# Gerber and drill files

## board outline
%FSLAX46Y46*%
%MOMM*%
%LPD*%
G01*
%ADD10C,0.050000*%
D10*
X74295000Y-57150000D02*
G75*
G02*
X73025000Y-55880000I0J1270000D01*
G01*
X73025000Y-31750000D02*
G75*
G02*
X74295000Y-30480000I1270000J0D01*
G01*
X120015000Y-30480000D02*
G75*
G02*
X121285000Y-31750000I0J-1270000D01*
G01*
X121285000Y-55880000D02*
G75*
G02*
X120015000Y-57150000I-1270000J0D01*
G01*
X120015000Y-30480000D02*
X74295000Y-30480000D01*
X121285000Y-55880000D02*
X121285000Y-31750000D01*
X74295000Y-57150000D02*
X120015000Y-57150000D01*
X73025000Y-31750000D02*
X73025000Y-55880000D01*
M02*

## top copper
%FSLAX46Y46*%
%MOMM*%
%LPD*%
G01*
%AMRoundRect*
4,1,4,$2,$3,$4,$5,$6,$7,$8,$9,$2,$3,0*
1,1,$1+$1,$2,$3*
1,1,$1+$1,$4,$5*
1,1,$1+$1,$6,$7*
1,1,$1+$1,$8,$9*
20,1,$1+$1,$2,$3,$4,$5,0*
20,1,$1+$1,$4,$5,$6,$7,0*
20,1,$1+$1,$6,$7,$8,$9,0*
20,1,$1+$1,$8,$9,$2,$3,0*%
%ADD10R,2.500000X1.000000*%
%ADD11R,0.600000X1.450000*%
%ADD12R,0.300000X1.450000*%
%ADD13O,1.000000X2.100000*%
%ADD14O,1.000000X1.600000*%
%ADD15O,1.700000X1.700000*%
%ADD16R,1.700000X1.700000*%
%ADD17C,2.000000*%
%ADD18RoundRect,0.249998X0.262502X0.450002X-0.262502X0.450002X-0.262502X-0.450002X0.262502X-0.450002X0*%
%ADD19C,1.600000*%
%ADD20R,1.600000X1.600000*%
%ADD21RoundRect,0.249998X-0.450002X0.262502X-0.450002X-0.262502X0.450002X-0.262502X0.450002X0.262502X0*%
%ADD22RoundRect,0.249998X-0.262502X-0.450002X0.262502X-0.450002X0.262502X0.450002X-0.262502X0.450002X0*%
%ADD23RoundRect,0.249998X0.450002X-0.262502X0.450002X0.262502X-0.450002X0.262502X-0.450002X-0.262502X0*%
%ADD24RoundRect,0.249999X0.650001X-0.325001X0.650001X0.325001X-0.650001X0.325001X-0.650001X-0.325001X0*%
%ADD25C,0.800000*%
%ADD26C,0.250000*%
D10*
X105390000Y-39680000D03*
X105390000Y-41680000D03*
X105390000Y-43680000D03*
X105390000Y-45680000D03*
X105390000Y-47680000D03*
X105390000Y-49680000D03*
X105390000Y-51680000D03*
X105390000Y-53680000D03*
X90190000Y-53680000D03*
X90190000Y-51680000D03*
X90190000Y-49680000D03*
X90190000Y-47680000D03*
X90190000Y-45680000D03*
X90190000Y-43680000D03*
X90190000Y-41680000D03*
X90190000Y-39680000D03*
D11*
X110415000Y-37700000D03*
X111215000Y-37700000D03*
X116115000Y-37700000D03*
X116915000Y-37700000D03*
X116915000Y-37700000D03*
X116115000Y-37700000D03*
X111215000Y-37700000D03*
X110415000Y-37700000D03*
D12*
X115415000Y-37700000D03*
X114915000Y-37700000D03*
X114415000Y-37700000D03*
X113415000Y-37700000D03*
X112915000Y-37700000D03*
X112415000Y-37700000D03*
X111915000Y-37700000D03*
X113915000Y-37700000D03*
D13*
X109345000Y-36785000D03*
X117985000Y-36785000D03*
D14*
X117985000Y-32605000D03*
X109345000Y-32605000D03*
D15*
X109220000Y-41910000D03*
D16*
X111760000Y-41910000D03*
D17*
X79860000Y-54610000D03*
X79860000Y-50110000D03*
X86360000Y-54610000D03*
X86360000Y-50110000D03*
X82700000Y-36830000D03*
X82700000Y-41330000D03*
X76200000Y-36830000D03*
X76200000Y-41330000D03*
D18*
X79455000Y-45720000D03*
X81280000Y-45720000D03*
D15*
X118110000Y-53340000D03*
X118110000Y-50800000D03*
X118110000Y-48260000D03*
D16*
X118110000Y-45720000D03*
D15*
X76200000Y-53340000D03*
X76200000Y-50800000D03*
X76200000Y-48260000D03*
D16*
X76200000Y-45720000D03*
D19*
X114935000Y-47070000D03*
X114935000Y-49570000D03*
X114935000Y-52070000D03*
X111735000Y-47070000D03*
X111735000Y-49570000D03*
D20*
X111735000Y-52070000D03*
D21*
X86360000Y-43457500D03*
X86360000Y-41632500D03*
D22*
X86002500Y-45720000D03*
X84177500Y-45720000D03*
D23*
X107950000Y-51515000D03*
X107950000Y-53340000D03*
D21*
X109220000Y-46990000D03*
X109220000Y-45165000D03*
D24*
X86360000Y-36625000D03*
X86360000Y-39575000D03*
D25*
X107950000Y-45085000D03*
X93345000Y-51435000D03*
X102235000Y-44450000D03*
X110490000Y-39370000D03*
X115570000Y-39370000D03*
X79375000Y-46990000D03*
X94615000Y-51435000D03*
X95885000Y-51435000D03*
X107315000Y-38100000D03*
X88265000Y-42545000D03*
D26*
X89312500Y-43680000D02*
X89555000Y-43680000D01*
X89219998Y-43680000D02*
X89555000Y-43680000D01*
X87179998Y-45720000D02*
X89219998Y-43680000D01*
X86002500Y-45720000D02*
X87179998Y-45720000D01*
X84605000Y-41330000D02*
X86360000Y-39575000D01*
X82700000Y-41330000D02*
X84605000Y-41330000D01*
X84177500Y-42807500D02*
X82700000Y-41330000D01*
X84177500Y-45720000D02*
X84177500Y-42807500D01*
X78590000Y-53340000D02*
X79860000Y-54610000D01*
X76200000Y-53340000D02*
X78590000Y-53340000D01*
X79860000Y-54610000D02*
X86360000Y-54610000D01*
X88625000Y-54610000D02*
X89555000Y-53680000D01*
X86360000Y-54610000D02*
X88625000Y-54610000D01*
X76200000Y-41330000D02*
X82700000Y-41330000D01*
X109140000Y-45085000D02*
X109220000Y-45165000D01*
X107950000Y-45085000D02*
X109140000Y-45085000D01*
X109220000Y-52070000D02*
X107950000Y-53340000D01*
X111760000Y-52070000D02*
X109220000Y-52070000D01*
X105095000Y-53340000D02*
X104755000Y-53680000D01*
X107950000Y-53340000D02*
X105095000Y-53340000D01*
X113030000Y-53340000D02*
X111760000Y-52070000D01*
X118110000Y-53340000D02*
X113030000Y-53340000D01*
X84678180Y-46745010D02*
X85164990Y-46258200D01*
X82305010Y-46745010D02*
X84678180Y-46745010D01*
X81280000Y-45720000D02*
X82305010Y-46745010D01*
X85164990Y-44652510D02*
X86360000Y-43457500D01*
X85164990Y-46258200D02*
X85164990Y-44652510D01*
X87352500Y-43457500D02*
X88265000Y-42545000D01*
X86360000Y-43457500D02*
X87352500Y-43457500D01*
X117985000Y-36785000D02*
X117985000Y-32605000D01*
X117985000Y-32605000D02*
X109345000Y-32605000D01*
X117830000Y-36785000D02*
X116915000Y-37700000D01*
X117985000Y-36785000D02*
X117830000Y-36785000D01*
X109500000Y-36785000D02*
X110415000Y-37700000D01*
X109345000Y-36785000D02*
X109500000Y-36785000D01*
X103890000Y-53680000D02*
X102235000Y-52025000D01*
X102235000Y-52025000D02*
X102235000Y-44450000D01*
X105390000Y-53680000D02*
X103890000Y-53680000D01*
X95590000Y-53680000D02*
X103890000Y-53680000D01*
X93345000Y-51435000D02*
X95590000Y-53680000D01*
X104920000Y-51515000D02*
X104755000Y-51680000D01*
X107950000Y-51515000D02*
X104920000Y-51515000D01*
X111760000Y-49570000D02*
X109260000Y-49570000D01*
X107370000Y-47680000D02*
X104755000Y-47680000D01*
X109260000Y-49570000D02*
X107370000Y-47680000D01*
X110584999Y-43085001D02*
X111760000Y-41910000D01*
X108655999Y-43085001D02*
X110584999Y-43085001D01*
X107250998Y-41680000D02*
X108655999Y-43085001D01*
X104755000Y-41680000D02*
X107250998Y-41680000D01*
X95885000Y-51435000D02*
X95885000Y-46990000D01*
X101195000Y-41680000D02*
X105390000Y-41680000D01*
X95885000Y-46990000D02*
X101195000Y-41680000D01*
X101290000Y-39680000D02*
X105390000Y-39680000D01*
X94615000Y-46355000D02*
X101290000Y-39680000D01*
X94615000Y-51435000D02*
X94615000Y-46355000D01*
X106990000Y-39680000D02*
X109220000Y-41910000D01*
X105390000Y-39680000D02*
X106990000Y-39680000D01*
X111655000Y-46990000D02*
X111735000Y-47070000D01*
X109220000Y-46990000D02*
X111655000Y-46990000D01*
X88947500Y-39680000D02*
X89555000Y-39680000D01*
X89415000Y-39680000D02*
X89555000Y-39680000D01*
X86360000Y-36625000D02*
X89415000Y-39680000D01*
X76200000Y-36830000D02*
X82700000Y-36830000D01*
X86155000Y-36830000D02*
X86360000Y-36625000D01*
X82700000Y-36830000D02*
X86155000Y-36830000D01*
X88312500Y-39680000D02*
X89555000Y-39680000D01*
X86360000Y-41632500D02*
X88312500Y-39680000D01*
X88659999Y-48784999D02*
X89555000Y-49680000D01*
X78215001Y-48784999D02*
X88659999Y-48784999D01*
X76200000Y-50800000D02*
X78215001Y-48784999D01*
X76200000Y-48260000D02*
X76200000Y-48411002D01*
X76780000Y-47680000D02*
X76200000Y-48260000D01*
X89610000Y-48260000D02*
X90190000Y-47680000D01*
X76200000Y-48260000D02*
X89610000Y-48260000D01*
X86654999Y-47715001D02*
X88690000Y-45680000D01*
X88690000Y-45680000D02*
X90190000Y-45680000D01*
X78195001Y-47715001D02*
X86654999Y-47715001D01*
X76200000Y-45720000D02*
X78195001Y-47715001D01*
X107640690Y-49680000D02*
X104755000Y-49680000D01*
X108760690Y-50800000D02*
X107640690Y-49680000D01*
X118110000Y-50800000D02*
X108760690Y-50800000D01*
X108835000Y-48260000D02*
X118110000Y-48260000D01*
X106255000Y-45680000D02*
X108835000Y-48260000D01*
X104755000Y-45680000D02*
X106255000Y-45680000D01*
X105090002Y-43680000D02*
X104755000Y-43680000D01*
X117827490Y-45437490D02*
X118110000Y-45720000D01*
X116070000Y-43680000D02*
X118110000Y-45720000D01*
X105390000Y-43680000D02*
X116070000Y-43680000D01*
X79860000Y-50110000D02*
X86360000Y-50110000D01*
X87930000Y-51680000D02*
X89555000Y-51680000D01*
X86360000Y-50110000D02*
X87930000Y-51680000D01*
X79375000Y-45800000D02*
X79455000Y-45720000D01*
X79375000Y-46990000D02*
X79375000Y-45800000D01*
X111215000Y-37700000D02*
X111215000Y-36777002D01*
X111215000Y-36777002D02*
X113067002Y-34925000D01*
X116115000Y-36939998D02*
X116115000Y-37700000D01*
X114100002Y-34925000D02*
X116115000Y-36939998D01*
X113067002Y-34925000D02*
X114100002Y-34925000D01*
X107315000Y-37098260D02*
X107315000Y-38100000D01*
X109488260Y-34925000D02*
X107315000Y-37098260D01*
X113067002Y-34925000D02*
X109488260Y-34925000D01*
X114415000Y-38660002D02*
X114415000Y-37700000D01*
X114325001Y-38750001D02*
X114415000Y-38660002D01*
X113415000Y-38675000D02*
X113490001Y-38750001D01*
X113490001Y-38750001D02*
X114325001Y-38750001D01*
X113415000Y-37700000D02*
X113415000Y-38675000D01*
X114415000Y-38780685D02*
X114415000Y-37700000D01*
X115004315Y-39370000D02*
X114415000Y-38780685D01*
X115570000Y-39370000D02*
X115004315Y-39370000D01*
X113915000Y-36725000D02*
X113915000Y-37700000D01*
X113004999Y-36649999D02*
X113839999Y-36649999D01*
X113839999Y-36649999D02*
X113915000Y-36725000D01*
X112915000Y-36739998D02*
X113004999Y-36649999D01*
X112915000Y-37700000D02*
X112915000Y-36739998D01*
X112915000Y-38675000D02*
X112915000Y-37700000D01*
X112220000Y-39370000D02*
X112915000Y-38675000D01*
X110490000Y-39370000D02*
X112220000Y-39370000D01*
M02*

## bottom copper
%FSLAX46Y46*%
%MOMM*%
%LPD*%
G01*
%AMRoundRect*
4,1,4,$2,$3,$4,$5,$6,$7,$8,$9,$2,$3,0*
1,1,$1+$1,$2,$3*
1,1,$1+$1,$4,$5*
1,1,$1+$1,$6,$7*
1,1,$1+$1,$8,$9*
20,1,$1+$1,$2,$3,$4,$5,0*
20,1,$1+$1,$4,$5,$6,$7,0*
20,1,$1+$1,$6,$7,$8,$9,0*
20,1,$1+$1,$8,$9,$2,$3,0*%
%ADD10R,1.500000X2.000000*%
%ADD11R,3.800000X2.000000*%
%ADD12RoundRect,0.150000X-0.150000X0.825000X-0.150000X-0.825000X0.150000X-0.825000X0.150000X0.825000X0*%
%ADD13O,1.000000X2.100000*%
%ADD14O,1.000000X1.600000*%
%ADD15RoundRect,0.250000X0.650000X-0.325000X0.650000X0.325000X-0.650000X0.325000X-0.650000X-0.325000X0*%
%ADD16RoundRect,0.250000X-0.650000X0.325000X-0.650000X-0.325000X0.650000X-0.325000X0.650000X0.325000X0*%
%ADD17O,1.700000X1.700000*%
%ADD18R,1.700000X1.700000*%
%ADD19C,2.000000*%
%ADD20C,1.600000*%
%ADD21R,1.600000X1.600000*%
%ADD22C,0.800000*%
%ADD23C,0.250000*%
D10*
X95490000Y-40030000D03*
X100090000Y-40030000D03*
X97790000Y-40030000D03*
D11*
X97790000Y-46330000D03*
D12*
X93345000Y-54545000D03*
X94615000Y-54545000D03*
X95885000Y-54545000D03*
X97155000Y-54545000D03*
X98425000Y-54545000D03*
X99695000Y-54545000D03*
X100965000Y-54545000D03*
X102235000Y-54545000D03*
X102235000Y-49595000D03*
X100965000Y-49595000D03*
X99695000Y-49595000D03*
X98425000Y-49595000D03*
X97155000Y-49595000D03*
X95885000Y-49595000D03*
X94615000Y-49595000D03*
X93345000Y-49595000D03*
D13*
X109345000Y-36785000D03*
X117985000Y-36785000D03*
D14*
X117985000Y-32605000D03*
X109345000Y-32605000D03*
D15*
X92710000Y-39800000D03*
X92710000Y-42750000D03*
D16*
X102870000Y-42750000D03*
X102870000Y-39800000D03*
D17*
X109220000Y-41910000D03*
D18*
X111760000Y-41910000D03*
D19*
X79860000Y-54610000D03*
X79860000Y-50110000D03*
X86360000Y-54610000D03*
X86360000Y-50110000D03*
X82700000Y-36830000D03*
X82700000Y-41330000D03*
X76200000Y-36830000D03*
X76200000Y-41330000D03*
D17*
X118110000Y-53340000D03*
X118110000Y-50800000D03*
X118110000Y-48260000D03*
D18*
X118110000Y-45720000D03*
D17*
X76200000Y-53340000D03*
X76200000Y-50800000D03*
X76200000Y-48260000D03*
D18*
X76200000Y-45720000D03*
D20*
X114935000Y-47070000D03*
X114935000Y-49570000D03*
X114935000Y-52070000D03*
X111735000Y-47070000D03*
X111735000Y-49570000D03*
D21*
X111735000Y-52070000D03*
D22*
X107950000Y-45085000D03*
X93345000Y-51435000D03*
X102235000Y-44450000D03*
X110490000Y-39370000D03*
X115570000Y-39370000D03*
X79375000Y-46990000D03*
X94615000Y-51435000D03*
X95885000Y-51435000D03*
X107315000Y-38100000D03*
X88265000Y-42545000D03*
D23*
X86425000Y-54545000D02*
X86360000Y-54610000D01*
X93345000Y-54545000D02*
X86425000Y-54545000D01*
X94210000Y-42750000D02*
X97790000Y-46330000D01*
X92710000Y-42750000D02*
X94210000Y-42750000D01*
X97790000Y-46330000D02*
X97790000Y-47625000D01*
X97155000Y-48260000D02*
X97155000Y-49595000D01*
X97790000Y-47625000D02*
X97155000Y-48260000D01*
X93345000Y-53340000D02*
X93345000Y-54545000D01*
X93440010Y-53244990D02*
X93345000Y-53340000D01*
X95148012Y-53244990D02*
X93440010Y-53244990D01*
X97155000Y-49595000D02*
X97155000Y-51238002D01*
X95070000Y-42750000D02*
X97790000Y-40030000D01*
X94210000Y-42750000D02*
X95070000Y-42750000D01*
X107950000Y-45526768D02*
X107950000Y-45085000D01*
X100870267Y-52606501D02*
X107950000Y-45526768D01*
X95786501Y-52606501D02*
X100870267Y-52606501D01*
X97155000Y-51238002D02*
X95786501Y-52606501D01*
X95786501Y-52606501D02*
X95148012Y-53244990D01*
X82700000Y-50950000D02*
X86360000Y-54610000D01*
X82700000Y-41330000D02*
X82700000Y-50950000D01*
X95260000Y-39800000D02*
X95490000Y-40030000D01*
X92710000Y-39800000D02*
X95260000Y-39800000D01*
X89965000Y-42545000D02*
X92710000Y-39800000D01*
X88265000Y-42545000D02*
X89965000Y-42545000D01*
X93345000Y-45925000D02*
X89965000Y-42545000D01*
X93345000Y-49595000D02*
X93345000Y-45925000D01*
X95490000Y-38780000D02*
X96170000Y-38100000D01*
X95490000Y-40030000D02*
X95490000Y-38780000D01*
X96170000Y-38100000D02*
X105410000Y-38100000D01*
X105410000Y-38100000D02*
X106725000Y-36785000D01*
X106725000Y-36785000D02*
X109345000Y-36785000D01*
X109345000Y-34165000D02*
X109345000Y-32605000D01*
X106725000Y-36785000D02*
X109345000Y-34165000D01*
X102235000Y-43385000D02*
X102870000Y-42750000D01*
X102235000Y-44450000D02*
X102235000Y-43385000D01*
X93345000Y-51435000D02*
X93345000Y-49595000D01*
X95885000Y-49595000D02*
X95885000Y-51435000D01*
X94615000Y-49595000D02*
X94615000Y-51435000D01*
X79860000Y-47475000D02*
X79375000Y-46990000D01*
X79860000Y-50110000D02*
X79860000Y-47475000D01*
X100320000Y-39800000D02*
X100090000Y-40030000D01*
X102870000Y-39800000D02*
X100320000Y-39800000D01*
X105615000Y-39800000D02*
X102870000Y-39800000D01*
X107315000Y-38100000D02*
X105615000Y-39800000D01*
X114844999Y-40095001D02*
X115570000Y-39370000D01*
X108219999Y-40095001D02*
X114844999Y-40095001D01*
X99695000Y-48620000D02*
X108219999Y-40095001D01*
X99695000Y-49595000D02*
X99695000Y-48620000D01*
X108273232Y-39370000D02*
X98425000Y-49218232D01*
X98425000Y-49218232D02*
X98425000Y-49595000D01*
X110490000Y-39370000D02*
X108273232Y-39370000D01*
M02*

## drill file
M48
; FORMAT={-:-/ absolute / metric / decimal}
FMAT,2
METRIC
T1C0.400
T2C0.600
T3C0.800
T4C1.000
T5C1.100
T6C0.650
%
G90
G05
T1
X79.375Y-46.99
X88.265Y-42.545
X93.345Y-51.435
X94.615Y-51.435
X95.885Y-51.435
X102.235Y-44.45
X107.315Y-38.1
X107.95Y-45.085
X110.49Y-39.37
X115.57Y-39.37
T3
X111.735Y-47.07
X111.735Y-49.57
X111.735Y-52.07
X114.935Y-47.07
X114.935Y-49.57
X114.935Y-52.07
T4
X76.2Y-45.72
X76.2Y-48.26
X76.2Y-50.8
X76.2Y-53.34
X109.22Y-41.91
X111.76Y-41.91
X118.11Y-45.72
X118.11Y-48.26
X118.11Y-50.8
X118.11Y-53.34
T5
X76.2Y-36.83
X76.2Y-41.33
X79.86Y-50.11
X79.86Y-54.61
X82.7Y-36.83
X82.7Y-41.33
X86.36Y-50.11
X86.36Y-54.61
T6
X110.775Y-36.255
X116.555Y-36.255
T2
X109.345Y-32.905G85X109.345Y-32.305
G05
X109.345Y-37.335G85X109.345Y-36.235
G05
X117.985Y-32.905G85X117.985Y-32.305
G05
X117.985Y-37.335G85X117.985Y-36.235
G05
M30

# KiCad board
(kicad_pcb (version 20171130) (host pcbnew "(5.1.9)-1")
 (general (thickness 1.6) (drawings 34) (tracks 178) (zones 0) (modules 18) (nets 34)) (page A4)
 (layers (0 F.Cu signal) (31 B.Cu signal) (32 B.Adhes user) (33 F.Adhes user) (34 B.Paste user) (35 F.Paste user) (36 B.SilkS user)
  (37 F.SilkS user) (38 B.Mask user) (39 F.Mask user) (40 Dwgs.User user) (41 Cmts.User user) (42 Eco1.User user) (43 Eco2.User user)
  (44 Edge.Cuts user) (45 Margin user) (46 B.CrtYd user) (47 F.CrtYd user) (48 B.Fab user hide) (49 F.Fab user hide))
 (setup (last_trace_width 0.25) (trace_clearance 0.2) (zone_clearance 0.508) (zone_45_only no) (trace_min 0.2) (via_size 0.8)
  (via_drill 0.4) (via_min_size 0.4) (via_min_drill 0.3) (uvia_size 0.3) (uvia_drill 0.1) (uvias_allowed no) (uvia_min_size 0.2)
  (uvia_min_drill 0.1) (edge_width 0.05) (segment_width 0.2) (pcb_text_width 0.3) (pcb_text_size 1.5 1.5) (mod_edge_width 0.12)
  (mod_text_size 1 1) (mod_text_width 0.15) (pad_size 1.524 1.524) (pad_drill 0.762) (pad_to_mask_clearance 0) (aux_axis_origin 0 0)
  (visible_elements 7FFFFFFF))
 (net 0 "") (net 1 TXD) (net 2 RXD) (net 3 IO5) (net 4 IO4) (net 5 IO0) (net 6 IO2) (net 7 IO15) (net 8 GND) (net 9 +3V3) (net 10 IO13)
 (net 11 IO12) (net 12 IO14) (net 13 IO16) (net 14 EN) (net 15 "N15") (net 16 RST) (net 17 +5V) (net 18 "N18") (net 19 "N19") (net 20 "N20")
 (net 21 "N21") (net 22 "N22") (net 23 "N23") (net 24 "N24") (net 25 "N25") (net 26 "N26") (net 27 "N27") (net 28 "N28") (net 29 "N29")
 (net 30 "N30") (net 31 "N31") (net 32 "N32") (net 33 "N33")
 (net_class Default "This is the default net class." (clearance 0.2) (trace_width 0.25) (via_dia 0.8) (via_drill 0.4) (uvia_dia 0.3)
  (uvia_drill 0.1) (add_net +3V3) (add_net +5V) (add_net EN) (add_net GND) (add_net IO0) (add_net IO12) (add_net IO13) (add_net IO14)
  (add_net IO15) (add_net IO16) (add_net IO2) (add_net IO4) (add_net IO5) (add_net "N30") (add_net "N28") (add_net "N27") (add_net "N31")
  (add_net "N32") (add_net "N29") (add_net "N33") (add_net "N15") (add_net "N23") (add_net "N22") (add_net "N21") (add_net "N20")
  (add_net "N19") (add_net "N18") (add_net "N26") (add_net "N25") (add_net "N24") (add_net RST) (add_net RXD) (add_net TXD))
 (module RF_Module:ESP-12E (layer F.Cu) (at 97.79 43.18)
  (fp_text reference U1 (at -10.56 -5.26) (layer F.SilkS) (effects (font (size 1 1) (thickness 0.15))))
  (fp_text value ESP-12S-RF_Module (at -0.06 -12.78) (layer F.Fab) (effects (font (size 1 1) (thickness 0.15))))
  (pad 16 smd rect (at 7.6 -3.5) (size 2.5 1) (layers F.Cu F.Paste F.Mask) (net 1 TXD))
  (pad 15 smd rect (at 7.6 -1.5) (size 2.5 1) (layers F.Cu F.Paste F.Mask) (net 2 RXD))
  (pad 14 smd rect (at 7.6 0.5) (size 2.5 1) (layers F.Cu F.Paste F.Mask) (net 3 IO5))
  (pad 13 smd rect (at 7.6 2.5) (size 2.5 1) (layers F.Cu F.Paste F.Mask) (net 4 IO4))
  (pad 12 smd rect (at 7.6 4.5) (size 2.5 1) (layers F.Cu F.Paste F.Mask) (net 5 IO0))
  (pad 11 smd rect (at 7.6 6.5) (size 2.5 1) (layers F.Cu F.Paste F.Mask) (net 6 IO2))
  (pad 10 smd rect (at 7.6 8.5) (size 2.5 1) (layers F.Cu F.Paste F.Mask) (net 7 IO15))
  (pad 9 smd rect (at 7.6 10.5) (size 2.5 1) (layers F.Cu F.Paste F.Mask) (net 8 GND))
  (pad 8 smd rect (at -7.6 10.5) (size 2.5 1) (layers F.Cu F.Paste F.Mask) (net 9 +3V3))
  (pad 7 smd rect (at -7.6 8.5) (size 2.5 1) (layers F.Cu F.Paste F.Mask) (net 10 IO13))
  (pad 6 smd rect (at -7.6 6.5) (size 2.5 1) (layers F.Cu F.Paste F.Mask) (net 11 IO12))
  (pad 5 smd rect (at -7.6 4.5) (size 2.5 1) (layers F.Cu F.Paste F.Mask) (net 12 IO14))
  (pad 4 smd rect (at -7.6 2.5) (size 2.5 1) (layers F.Cu F.Paste F.Mask) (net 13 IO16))
  (pad 3 smd rect (at -7.6 0.5) (size 2.5 1) (layers F.Cu F.Paste F.Mask) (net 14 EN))
  (pad 2 smd rect (at -7.6 -1.5) (size 2.5 1) (layers F.Cu F.Paste F.Mask) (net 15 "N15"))
  (pad 1 smd rect (at -7.6 -3.5) (size 2.5 1) (layers F.Cu F.Paste F.Mask) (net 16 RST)))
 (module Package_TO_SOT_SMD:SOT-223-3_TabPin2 (layer B.Cu) (at 97.79 43.18 270)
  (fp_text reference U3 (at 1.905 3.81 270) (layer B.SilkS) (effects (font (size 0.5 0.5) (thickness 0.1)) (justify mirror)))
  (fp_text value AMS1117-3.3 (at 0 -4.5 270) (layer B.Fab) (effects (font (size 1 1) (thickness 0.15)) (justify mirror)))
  (pad 1 smd rect (at -3.15 2.3 270) (size 2 1.5) (layers B.Cu B.Paste B.Mask) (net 8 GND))
  (pad 3 smd rect (at -3.15 -2.3 270) (size 2 1.5) (layers B.Cu B.Paste B.Mask) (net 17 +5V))
  (pad 2 smd rect (at -3.15 0 270) (size 2 1.5) (layers B.Cu B.Paste B.Mask) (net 9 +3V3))
  (pad 2 smd rect (at 3.15 0 270) (size 2 3.8) (layers B.Cu B.Paste B.Mask) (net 9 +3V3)))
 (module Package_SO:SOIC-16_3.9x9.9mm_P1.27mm (layer B.Cu) (at 97.79 52.07 270)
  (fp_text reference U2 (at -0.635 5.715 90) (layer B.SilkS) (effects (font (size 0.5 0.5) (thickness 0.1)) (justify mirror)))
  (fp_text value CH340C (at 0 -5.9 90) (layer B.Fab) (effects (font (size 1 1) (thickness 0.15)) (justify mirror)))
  (pad 16 smd roundrect (at 2.475 4.445 270) (size 1.95 0.6) (layers B.Cu B.Paste B.Mask) (roundrect_rratio 0.25) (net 9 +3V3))
  (pad 15 smd roundrect (at 2.475 3.175 270) (size 1.95 0.6) (layers B.Cu B.Paste B.Mask) (roundrect_rratio 0.25) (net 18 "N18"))
  (pad 14 smd roundrect (at 2.475 1.905 270) (size 1.95 0.6) (layers B.Cu B.Paste B.Mask) (roundrect_rratio 0.25) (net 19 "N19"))
  (pad 13 smd roundrect (at 2.475 0.635 270) (size 1.95 0.6) (layers B.Cu B.Paste B.Mask) (roundrect_rratio 0.25) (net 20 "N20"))
  (pad 12 smd roundrect (at 2.475 -0.635 270) (size 1.95 0.6) (layers B.Cu B.Paste B.Mask) (roundrect_rratio 0.25) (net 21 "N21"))
  (pad 11 smd roundrect (at 2.475 -1.905 270) (size 1.95 0.6) (layers B.Cu B.Paste B.Mask) (roundrect_rratio 0.25) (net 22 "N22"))
  (pad 10 smd roundrect (at 2.475 -3.175 270) (size 1.95 0.6) (layers B.Cu B.Paste B.Mask) (roundrect_rratio 0.25) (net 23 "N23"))
  (pad 9 smd roundrect (at 2.475 -4.445 270) (size 1.95 0.6) (layers B.Cu B.Paste B.Mask) (roundrect_rratio 0.25) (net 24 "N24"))
  (pad 8 smd roundrect (at -2.475 -4.445 270) (size 1.95 0.6) (layers B.Cu B.Paste B.Mask) (roundrect_rratio 0.25) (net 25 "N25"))
  (pad 7 smd roundrect (at -2.475 -3.175 270) (size 1.95 0.6) (layers B.Cu B.Paste B.Mask) (roundrect_rratio 0.25) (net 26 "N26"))
  (pad 6 smd roundrect (at -2.475 -1.905 270) (size 1.95 0.6) (layers B.Cu B.Paste B.Mask) (roundrect_rratio 0.25) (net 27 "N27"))
  (pad 5 smd roundrect (at -2.475 -0.635 270) (size 1.95 0.6) (layers B.Cu B.Paste B.Mask) (roundrect_rratio 0.25) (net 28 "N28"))
  (pad 4 smd roundrect (at -2.475 0.635 270) (size 1.95 0.6) (layers B.Cu B.Paste B.Mask) (roundrect_rratio 0.25) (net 9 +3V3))
  (pad 3 smd roundrect (at -2.475 1.905 270) (size 1.95 0.6) (layers B.Cu B.Paste B.Mask) (roundrect_rratio 0.25) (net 2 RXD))
  (pad 2 smd roundrect (at -2.475 3.175 270) (size 1.95 0.6) (layers B.Cu B.Paste B.Mask) (roundrect_rratio 0.25) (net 1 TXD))
  (pad 1 smd roundrect (at -2.475 4.445 270) (size 1.95 0.6) (layers B.Cu B.Paste B.Mask) (roundrect_rratio 0.25) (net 8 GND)))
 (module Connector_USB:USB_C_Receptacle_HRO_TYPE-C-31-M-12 (layer F.Cu) (at 113.665 33.655 180)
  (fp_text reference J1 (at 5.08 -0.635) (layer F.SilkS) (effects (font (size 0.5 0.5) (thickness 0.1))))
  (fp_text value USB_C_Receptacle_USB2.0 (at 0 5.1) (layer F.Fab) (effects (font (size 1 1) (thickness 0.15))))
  (pad B1 smd rect (at 3.25 -4.045 180) (size 0.6 1.45) (layers F.Cu F.Paste F.Mask) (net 8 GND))
  (pad A9 smd rect (at 2.45 -4.045 180) (size 0.6 1.45) (layers F.Cu F.Paste F.Mask) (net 17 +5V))
  (pad B9 smd rect (at -2.45 -4.045 180) (size 0.6 1.45) (layers F.Cu F.Paste F.Mask) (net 17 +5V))
  (pad B12 smd rect (at -3.25 -4.045 180) (size 0.6 1.45) (layers F.Cu F.Paste F.Mask) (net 8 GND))
  (pad A1 smd rect (at -3.25 -4.045 180) (size 0.6 1.45) (layers F.Cu F.Paste F.Mask) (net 8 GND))
  (pad A4 smd rect (at -2.45 -4.045 180) (size 0.6 1.45) (layers F.Cu F.Paste F.Mask) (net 17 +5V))
  (pad B4 smd rect (at 2.45 -4.045 180) (size 0.6 1.45) (layers F.Cu F.Paste F.Mask) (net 17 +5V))
  (pad A12 smd rect (at 3.25 -4.045 180) (size 0.6 1.45) (layers F.Cu F.Paste F.Mask) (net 8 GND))
  (pad B8 smd rect (at -1.75 -4.045 180) (size 0.3 1.45) (layers F.Cu F.Paste F.Mask) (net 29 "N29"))
  (pad A5 smd rect (at -1.25 -4.045 180) (size 0.3 1.45) (layers F.Cu F.Paste F.Mask) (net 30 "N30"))
  (pad B7 smd rect (at -0.75 -4.045 180) (size 0.3 1.45) (layers F.Cu F.Paste F.Mask) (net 27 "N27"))
  (pad A7 smd rect (at 0.25 -4.045 180) (size 0.3 1.45) (layers F.Cu F.Paste F.Mask) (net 27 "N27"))
  (pad B6 smd rect (at 0.75 -4.045 180) (size 0.3 1.45) (layers F.Cu F.Paste F.Mask) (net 28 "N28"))
  (pad A8 smd rect (at 1.25 -4.045 180) (size 0.3 1.45) (layers F.Cu F.Paste F.Mask) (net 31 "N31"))
  (pad B5 smd rect (at 1.75 -4.045 180) (size 0.3 1.45) (layers F.Cu F.Paste F.Mask) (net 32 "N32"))
  (pad A6 smd rect (at -0.25 -4.045 180) (size 0.3 1.45) (layers F.Cu F.Paste F.Mask) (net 28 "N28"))
  (pad S1 thru_hole oval (at 4.32 -3.13 180) (size 1 2.1) (drill oval 0.6 1.7) (layers *.Cu *.Mask) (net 8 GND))
  (pad S1 thru_hole oval (at -4.32 -3.13 180) (size 1 2.1) (drill oval 0.6 1.7) (layers *.Cu *.Mask) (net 8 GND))
  (pad "" np_thru_hole circle (at -2.89 -2.6 180) (size 0.65 0.65) (drill 0.65) (layers *.Cu *.Mask))
  (pad S1 thru_hole oval (at -4.32 1.05 180) (size 1 1.6) (drill oval 0.6 1.2) (layers *.Cu *.Mask) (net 8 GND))
  (pad "" np_thru_hole circle (at 2.89 -2.6 180) (size 0.65 0.65) (drill 0.65) (layers *.Cu *.Mask))
  (pad S1 thru_hole oval (at 4.32 1.05 180) (size 1 1.6) (drill oval 0.6 1.2) (layers *.Cu *.Mask) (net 8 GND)))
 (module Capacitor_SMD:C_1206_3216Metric (layer B.Cu) (at 92.71 41.275 90)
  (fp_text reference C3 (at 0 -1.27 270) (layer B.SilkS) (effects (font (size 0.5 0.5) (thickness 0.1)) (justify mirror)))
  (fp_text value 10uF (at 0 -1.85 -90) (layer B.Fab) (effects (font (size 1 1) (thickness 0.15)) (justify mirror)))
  (pad 2 smd roundrect (at 1.475 0 90) (size 1.15 1.8) (layers B.Cu B.Paste B.Mask) (roundrect_rratio 0.217391) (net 8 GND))
  (pad 1 smd roundrect (at -1.475 0 90) (size 1.15 1.8) (layers B.Cu B.Paste B.Mask) (roundrect_rratio 0.217391) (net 9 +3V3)))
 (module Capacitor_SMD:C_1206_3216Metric (layer B.Cu) (at 102.87 41.275 270)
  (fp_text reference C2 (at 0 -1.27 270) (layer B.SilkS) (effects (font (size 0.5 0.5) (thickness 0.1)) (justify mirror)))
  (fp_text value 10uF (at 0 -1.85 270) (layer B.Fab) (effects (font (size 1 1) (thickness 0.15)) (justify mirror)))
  (pad 2 smd roundrect (at 1.475 0 270) (size 1.15 1.8) (layers B.Cu B.Paste B.Mask) (roundrect_rratio 0.217391) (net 8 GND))
  (pad 1 smd roundrect (at -1.475 0 270) (size 1.15 1.8) (layers B.Cu B.Paste B.Mask) (roundrect_rratio 0.217391) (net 17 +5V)))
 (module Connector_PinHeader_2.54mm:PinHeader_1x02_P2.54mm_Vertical (layer B.Cu) (at 111.76 41.91 90)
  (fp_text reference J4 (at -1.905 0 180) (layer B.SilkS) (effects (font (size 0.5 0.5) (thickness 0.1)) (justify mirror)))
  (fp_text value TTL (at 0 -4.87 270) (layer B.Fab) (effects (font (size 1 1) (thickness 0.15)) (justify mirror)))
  (pad 2 thru_hole oval (at 0 -2.54 90) (size 1.7 1.7) (drill 1) (layers *.Cu *.Mask) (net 1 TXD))
  (pad 1 thru_hole rect (at 0 0 90) (size 1.7 1.7) (drill 1) (layers *.Cu *.Mask) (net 2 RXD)))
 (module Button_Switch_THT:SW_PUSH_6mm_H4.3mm (layer F.Cu) (at 86.36 54.61 180)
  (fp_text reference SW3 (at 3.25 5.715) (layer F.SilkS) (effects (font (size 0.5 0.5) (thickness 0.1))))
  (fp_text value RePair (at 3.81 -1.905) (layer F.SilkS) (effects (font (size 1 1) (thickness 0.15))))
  (pad 1 thru_hole circle (at 6.5 0 270) (size 2 2) (drill 1.1) (layers *.Cu *.Mask) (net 9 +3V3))
  (pad 2 thru_hole circle (at 6.5 4.5 270) (size 2 2) (drill 1.1) (layers *.Cu *.Mask) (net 10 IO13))
  (pad 1 thru_hole circle (at 0 0 270) (size 2 2) (drill 1.1) (layers *.Cu *.Mask) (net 9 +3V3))
  (pad 2 thru_hole circle (at 0 4.5 270) (size 2 2) (drill 1.1) (layers *.Cu *.Mask) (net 10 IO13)))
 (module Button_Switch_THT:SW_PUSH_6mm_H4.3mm (layer F.Cu) (at 76.2 36.83)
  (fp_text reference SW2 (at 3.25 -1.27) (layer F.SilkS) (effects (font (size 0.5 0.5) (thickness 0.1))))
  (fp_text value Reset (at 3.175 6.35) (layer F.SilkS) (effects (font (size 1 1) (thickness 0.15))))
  (pad 1 thru_hole circle (at 6.5 0 90) (size 2 2) (drill 1.1) (layers *.Cu *.Mask) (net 16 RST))
  (pad 2 thru_hole circle (at 6.5 4.5 90) (size 2 2) (drill 1.1) (layers *.Cu *.Mask) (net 9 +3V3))
  (pad 1 thru_hole circle (at 0 0 90) (size 2 2) (drill 1.1) (layers *.Cu *.Mask) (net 16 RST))
  (pad 2 thru_hole circle (at 0 4.5 90) (size 2 2) (drill 1.1) (layers *.Cu *.Mask) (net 9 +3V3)))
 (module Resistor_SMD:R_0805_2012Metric (layer F.Cu) (at 80.3675 45.72 180)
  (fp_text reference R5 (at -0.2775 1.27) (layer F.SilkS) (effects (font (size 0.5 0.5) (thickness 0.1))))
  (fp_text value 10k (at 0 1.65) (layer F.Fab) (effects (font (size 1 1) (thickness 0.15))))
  (pad 2 smd roundrect (at 0.9125 0 180) (size 1.025 1.4) (layers F.Cu F.Paste F.Mask) (roundrect_rratio 0.2439004878048781) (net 10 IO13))
  (pad 1 smd roundrect (at -0.9125 0 180) (size 1.025 1.4) (layers F.Cu F.Paste F.Mask) (roundrect_rratio 0.2439004878048781) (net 8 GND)))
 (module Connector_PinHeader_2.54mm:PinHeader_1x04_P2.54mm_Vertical (layer B.Cu) (at 118.11 45.72 180)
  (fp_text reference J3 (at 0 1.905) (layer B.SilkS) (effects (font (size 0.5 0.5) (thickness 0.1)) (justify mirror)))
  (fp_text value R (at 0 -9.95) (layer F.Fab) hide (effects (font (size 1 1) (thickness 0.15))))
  (pad 4 thru_hole oval (at 0 -7.62 180) (size 1.7 1.7) (drill 1) (layers *.Cu *.Mask) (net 8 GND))
  (pad 3 thru_hole oval (at 0 -5.08 180) (size 1.7 1.7) (drill 1) (layers *.Cu *.Mask) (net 6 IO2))
  (pad 2 thru_hole oval (at 0 -2.54 180) (size 1.7 1.7) (drill 1) (layers *.Cu *.Mask) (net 4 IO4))
  (pad 1 thru_hole rect (at 0 0 180) (size 1.7 1.7) (drill 1) (layers *.Cu *.Mask) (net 3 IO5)))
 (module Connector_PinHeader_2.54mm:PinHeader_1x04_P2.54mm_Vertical (layer B.Cu) (at 76.2 45.72 180)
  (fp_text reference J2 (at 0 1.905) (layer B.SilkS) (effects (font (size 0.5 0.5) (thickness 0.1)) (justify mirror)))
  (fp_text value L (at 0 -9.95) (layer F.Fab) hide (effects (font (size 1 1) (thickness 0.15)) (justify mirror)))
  (pad 4 thru_hole oval (at 0 -7.62 180) (size 1.7 1.7) (drill 1) (layers *.Cu *.Mask) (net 9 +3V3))
  (pad 3 thru_hole oval (at 0 -5.08 180) (size 1.7 1.7) (drill 1) (layers *.Cu *.Mask) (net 11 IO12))
  (pad 2 thru_hole oval (at 0 -2.54 180) (size 1.7 1.7) (drill 1) (layers *.Cu *.Mask) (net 12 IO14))
  (pad 1 thru_hole rect (at 0 0 180) (size 1.7 1.7) (drill 1) (layers *.Cu *.Mask) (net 13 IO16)))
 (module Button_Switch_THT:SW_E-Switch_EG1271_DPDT (layer F.Cu) (at 111.735 52.07 90)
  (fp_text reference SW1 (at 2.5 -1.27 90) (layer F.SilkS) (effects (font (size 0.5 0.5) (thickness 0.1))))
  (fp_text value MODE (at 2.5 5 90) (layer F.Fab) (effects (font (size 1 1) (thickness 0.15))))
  (pad 6 thru_hole circle (at 5 3.2 90) (size 1.6 1.6) (drill 0.8) (layers *.Cu *.Mask))
  (pad 5 thru_hole circle (at 2.5 3.2 90) (size 1.6 1.6) (drill 0.8) (layers *.Cu *.Mask))
  (pad 4 thru_hole circle (at 0 3.2 90) (size 1.6 1.6) (drill 0.8) (layers *.Cu *.Mask))
  (pad 3 thru_hole circle (at 5 0 90) (size 1.6 1.6) (drill 0.8) (layers *.Cu *.Mask) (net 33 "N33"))
  (pad 2 thru_hole circle (at 2.5 0 90) (size 1.6 1.6) (drill 0.8) (layers *.Cu *.Mask) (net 5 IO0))
  (pad 1 thru_hole rect (at 0 0 90) (size 1.6 1.6) (drill 0.8) (layers *.Cu *.Mask) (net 8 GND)))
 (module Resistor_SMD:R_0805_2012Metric (layer F.Cu) (at 86.36 42.545 270)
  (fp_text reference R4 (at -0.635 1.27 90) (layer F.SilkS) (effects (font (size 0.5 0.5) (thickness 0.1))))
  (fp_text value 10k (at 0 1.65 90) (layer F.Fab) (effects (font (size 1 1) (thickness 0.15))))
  (pad 2 smd roundrect (at 0.9125 0 270) (size 1.025 1.4) (layers F.Cu F.Paste F.Mask) (roundrect_rratio 0.2439004878048781) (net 8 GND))
  (pad 1 smd roundrect (at -0.9125 0 270) (size 1.025 1.4) (layers F.Cu F.Paste F.Mask) (roundrect_rratio 0.2439004878048781) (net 16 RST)))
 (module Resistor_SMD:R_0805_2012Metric (layer F.Cu) (at 85.09 45.72)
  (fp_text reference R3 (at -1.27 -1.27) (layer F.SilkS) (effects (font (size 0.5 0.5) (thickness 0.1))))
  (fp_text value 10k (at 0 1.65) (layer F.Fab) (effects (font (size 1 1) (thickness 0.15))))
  (pad 2 smd roundrect (at 0.9125 0) (size 1.025 1.4) (layers F.Cu F.Paste F.Mask) (roundrect_rratio 0.2439004878048781) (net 14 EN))
  (pad 1 smd roundrect (at -0.9125 0) (size 1.025 1.4) (layers F.Cu F.Paste F.Mask) (roundrect_rratio 0.2439004878048781) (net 9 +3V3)))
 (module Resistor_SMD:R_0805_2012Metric (layer F.Cu) (at 107.95 52.4275 90)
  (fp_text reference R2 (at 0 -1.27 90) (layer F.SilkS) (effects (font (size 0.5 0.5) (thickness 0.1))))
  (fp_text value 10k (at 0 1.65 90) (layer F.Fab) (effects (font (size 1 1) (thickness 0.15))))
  (pad 2 smd roundrect (at 0.9125 0 90) (size 1.025 1.4) (layers F.Cu F.Paste F.Mask) (roundrect_rratio 0.2439004878048781) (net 7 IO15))
  (pad 1 smd roundrect (at -0.9125 0 90) (size 1.025 1.4) (layers F.Cu F.Paste F.Mask) (roundrect_rratio 0.2439004878048781) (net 8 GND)))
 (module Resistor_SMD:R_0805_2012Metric (layer F.Cu) (at 109.22 46.0775 270)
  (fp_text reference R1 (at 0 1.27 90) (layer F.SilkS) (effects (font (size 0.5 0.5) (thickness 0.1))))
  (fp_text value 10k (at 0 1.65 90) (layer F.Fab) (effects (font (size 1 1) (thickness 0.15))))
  (pad 2 smd roundrect (at 0.9125 0 270) (size 1.025 1.4) (layers F.Cu F.Paste F.Mask) (roundrect_rratio 0.2439004878048781) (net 33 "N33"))
  (pad 1 smd roundrect (at -0.9125 0 270) (size 1.025 1.4) (layers F.Cu F.Paste F.Mask) (roundrect_rratio 0.2439004878048781) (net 9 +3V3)))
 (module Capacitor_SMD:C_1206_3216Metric (layer F.Cu) (at 86.36 38.1 90)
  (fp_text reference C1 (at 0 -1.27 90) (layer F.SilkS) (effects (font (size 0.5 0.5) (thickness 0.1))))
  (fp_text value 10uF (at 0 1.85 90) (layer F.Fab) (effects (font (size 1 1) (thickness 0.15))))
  (pad 2 smd roundrect (at 1.475 0 90) (size 1.15 1.8) (layers F.Cu F.Paste F.Mask) (roundrect_rratio 0.2173904347826087) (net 16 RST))
  (pad 1 smd roundrect (at -1.475 0 90) (size 1.15 1.8) (layers F.Cu F.Paste F.Mask) (roundrect_rratio 0.2173904347826087) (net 9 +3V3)))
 (gr_arc (start 74.295 55.88) (end 73.025 55.88) (angle -90) (layer Edge.Cuts) (width 0.05))
 (gr_arc (start 74.295 31.75) (end 74.295 30.48) (angle -90) (layer Edge.Cuts) (width 0.05))
 (gr_arc (start 120.015 31.75) (end 121.285 31.75) (angle -90) (layer Edge.Cuts) (width 0.05))
 (gr_arc (start 120.015 55.88) (end 120.015 57.15) (angle -90) (layer Edge.Cuts) (width 0.05))
 (gr_line (start 120.015 30.48) (end 74.295 30.48) (layer Edge.Cuts) (width 0.05))
 (gr_line (start 121.285 55.88) (end 121.285 31.75) (layer Edge.Cuts) (width 0.05))
 (gr_line (start 74.295 57.15) (end 120.015 57.15) (layer Edge.Cuts) (width 0.05))
 (gr_line (start 73.025 31.75) (end 73.025 55.88) (layer Edge.Cuts) (width 0.05))
 (via (at 107.95 45.085) (size 0.8) (drill 0.4) (layers F.Cu B.Cu) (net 9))
 (via (at 93.345 51.435) (size 0.8) (drill 0.4) (layers F.Cu B.Cu) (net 8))
 (via (at 102.235 44.45) (size 0.8) (drill 0.4) (layers F.Cu B.Cu) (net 8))
 (via (at 110.49 39.37) (size 0.8) (drill 0.4) (layers F.Cu B.Cu) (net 28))
 (via (at 115.57 39.37) (size 0.8) (drill 0.4) (layers F.Cu B.Cu) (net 27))
 (via (at 79.375 46.99) (size 0.8) (drill 0.4) (layers F.Cu B.Cu) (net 10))
 (via (at 94.615 51.435) (size 0.8) (drill 0.4) (layers F.Cu B.Cu) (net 1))
 (via (at 95.885 51.435) (size 0.8) (drill 0.4) (layers F.Cu B.Cu) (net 2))
 (via (at 107.315 38.1) (size 0.8) (drill 0.4) (layers F.Cu B.Cu) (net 17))
 (via (at 88.265 42.545) (size 0.8) (drill 0.4) (layers F.Cu B.Cu) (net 8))
 (segment (start 89.3125 43.68) (end 89.555 43.68) (width 0.25) (layer F.Cu) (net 14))
 (segment (start 89.219998 43.68) (end 89.555 43.68) (width 0.25) (layer F.Cu) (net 14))
 (segment (start 87.179998 45.72) (end 89.219998 43.68) (width 0.25) (layer F.Cu) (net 14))
 (segment (start 86.0025 45.72) (end 87.179998 45.72) (width 0.25) (layer F.Cu) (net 14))
 (segment (start 84.605 41.33) (end 86.36 39.575) (width 0.25) (layer F.Cu) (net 9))
 (segment (start 82.7 41.33) (end 84.605 41.33) (width 0.25) (layer F.Cu) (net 9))
 (segment (start 84.1775 42.8075) (end 82.7 41.33) (width 0.25) (layer F.Cu) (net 9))
 (segment (start 84.1775 45.72) (end 84.1775 42.8075) (width 0.25) (layer F.Cu) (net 9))
 (segment (start 78.59 53.34) (end 79.86 54.61) (width 0.25) (layer F.Cu) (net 9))
 (segment (start 76.2 53.34) (end 78.59 53.34) (width 0.25) (layer F.Cu) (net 9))
 (segment (start 79.86 54.61) (end 86.36 54.61) (width 0.25) (layer F.Cu) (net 9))
 (segment (start 88.625 54.61) (end 89.555 53.68) (width 0.25) (layer F.Cu) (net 9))
 (segment (start 86.36 54.61) (end 88.625 54.61) (width 0.25) (layer F.Cu) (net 9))
 (segment (start 86.425 54.545) (end 86.36 54.61) (width 0.25) (layer B.Cu) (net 9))
 (segment (start 93.345 54.545) (end 86.425 54.545) (width 0.25) (layer B.Cu) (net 9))
 (segment (start 94.21 42.75) (end 97.79 46.33) (width 0.25) (layer B.Cu) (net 9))
 (segment (start 92.71 42.75) (end 94.21 42.75) (width 0.25) (layer B.Cu) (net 9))
 (segment (start 97.79 46.33) (end 97.79 47.625) (width 0.25) (layer B.Cu) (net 9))
 (segment (start 97.155 48.26) (end 97.155 49.595) (width 0.25) (layer B.Cu) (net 9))
 (segment (start 97.79 47.625) (end 97.155 48.26) (width 0.25) (layer B.Cu) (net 9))
 (segment (start 93.345 53.34) (end 93.345 54.545) (width 0.25) (layer B.Cu) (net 9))
 (segment (start 93.44001 53.24499) (end 93.345 53.34) (width 0.25) (layer B.Cu) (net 9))
 (segment (start 95.148012 53.24499) (end 93.44001 53.24499) (width 0.25) (layer B.Cu) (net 9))
 (segment (start 97.155 49.595) (end 97.155 51.238002) (width 0.25) (layer B.Cu) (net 9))
 (segment (start 95.07 42.75) (end 97.79 40.03) (width 0.25) (layer B.Cu) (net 9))
 (segment (start 94.21 42.75) (end 95.07 42.75) (width 0.25) (layer B.Cu) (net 9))
 (segment (start 76.2 41.33) (end 82.7 41.33) (width 0.25) (layer F.Cu) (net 9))
 (segment (start 107.95 45.526768) (end 107.95 45.085) (width 0.25) (layer B.Cu) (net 9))
 (segment (start 100.870267 52.606501) (end 107.95 45.526768) (width 0.25) (layer B.Cu) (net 9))
 (segment (start 95.786501 52.606501) (end 100.870267 52.606501) (width 0.25) (layer B.Cu) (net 9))
 (segment (start 97.155 51.238002) (end 95.786501 52.606501) (width 0.25) (layer B.Cu) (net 9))
 (segment (start 95.786501 52.606501) (end 95.148012 53.24499) (width 0.25) (layer B.Cu) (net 9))
 (segment (start 109.14 45.085) (end 109.22 45.165) (width 0.25) (layer F.Cu) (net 9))
 (segment (start 107.95 45.085) (end 109.14 45.085) (width 0.25) (layer F.Cu) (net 9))
 (segment (start 82.7 50.95) (end 86.36 54.61) (width 0.25) (layer B.Cu) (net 9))
 (segment (start 82.7 41.33) (end 82.7 50.95) (width 0.25) (layer B.Cu) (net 9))
 (segment (start 109.22 52.07) (end 107.95 53.34) (width 0.25) (layer F.Cu) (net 8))
 (segment (start 111.76 52.07) (end 109.22 52.07) (width 0.25) (layer F.Cu) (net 8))
 (segment (start 105.095 53.34) (end 104.755 53.68) (width 0.25) (layer F.Cu) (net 8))
 (segment (start 107.95 53.34) (end 105.095 53.34) (width 0.25) (layer F.Cu) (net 8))
 (segment (start 113.03 53.34) (end 111.76 52.07) (width 0.25) (layer F.Cu) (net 8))
 (segment (start 118.11 53.34) (end 113.03 53.34) (width 0.25) (layer F.Cu) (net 8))
 (segment (start 84.67818 46.74501) (end 85.16499 46.2582) (width 0.25) (layer F.Cu) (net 8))
 (segment (start 82.30501 46.74501) (end 84.67818 46.74501) (width 0.25) (layer F.Cu) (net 8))
 (segment (start 81.28 45.72) (end 82.30501 46.74501) (width 0.25) (layer F.Cu) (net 8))
 (segment (start 85.16499 44.65251) (end 86.36 43.4575) (width 0.25) (layer F.Cu) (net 8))
 (segment (start 85.16499 46.2582) (end 85.16499 44.65251) (width 0.25) (layer F.Cu) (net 8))
 (segment (start 95.26 39.8) (end 95.49 40.03) (width 0.25) (layer B.Cu) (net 8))
 (segment (start 92.71 39.8) (end 95.26 39.8) (width 0.25) (layer B.Cu) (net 8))
 (segment (start 87.3525 43.4575) (end 88.265 42.545) (width 0.25) (layer F.Cu) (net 8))
 (segment (start 86.36 43.4575) (end 87.3525 43.4575) (width 0.25) (layer F.Cu) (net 8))
 (segment (start 89.965 42.545) (end 92.71 39.8) (width 0.25) (layer B.Cu) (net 8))
 (segment (start 88.265 42.545) (end 89.965 42.545) (width 0.25) (layer B.Cu) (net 8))
 (segment (start 93.345 45.925) (end 89.965 42.545) (width 0.25) (layer B.Cu) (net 8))
 (segment (start 93.345 49.595) (end 93.345 45.925) (width 0.25) (layer B.Cu) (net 8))
 (segment (start 117.985 36.785) (end 117.985 32.605) (width 0.25) (layer F.Cu) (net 8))
 (segment (start 117.985 32.605) (end 109.345 32.605) (width 0.25) (layer F.Cu) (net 8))
 (segment (start 117.83 36.785) (end 116.915 37.7) (width 0.25) (layer F.Cu) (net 8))
 (segment (start 117.985 36.785) (end 117.83 36.785) (width 0.25) (layer F.Cu) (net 8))
 (segment (start 109.5 36.785) (end 110.415 37.7) (width 0.25) (layer F.Cu) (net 8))
 (segment (start 109.345 36.785) (end 109.5 36.785) (width 0.25) (layer F.Cu) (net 8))
 (segment (start 95.49 38.78) (end 96.17 38.1) (width 0.25) (layer B.Cu) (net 8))
 (segment (start 95.49 40.03) (end 95.49 38.78) (width 0.25) (layer B.Cu) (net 8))
 (segment (start 96.17 38.1) (end 105.41 38.1) (width 0.25) (layer B.Cu) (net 8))
 (segment (start 105.41 38.1) (end 106.725 36.785) (width 0.25) (layer B.Cu) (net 8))
 (segment (start 103.89 53.68) (end 102.235 52.025) (width 0.25) (layer F.Cu) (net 8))
 (segment (start 102.235 52.025) (end 102.235 44.45) (width 0.25) (layer F.Cu) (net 8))
 (segment (start 105.39 53.68) (end 103.89 53.68) (width 0.25) (layer F.Cu) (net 8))
 (segment (start 106.725 36.785) (end 109.345 36.785) (width 0.25) (layer B.Cu) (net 8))
 (segment (start 109.345 34.165) (end 109.345 32.605) (width 0.25) (layer B.Cu) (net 8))
 (segment (start 106.725 36.785) (end 109.345 34.165) (width 0.25) (layer B.Cu) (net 8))
 (segment (start 102.235 43.385) (end 102.87 42.75) (width 0.25) (layer B.Cu) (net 8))
 (segment (start 102.235 44.45) (end 102.235 43.385) (width 0.25) (layer B.Cu) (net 8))
 (segment (start 93.345 51.435) (end 93.345 49.595) (width 0.25) (layer B.Cu) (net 8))
 (segment (start 95.59 53.68) (end 103.89 53.68) (width 0.25) (layer F.Cu) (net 8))
 (segment (start 93.345 51.435) (end 95.59 53.68) (width 0.25) (layer F.Cu) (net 8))
 (segment (start 104.92 51.515) (end 104.755 51.68) (width 0.25) (layer F.Cu) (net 7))
 (segment (start 107.95 51.515) (end 104.92 51.515) (width 0.25) (layer F.Cu) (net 7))
 (segment (start 111.76 49.57) (end 109.26 49.57) (width 0.25) (layer F.Cu) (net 5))
 (segment (start 107.37 47.68) (end 104.755 47.68) (width 0.25) (layer F.Cu) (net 5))
 (segment (start 109.26 49.57) (end 107.37 47.68) (width 0.25) (layer F.Cu) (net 5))
 (segment (start 110.584999 43.085001) (end 111.76 41.91) (width 0.25) (layer F.Cu) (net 2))
 (segment (start 108.655999 43.085001) (end 110.584999 43.085001) (width 0.25) (layer F.Cu) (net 2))
 (segment (start 107.250998 41.68) (end 108.655999 43.085001) (width 0.25) (layer F.Cu) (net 2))
 (segment (start 104.755 41.68) (end 107.250998 41.68) (width 0.25) (layer F.Cu) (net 2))
 (segment (start 95.885 49.595) (end 95.885 51.435) (width 0.25) (layer B.Cu) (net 2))
 (segment (start 95.885 51.435) (end 95.885 46.99) (width 0.25) (layer F.Cu) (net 2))
 (segment (start 101.195 41.68) (end 105.39 41.68) (width 0.25) (layer F.Cu) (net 2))
 (segment (start 95.885 46.99) (end 101.195 41.68) (width 0.25) (layer F.Cu) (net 2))
 (segment (start 94.615 49.595) (end 94.615 51.435) (width 0.25) (layer B.Cu) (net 1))
 (segment (start 101.29 39.68) (end 105.39 39.68) (width 0.25) (layer F.Cu) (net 1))
 (segment (start 94.615 46.355) (end 101.29 39.68) (width 0.25) (layer F.Cu) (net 1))
 (segment (start 94.615 51.435) (end 94.615 46.355) (width 0.25) (layer F.Cu) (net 1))
 (segment (start 106.99 39.68) (end 109.22 41.91) (width 0.25) (layer F.Cu) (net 1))
 (segment (start 105.39 39.68) (end 106.99 39.68) (width 0.25) (layer F.Cu) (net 1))
 (segment (start 111.655 46.99) (end 111.735 47.07) (width 0.25) (layer F.Cu) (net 33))
 (segment (start 109.22 46.99) (end 111.655 46.99) (width 0.25) (layer F.Cu) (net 33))
 (segment (start 88.9475 39.68) (end 89.555 39.68) (width 0.25) (layer F.Cu) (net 16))
 (segment (start 89.415 39.68) (end 89.555 39.68) (width 0.25) (layer F.Cu) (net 16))
 (segment (start 86.36 36.625) (end 89.415 39.68) (width 0.25) (layer F.Cu) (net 16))
 (segment (start 76.2 36.83) (end 82.7 36.83) (width 0.25) (layer F.Cu) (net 16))
 (segment (start 86.155 36.83) (end 86.36 36.625) (width 0.25) (layer F.Cu) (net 16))
 (segment (start 82.7 36.83) (end 86.155 36.83) (width 0.25) (layer F.Cu) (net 16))
 (segment (start 88.3125 39.68) (end 89.555 39.68) (width 0.25) (layer F.Cu) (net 16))
 (segment (start 86.36 41.6325) (end 88.3125 39.68) (width 0.25) (layer F.Cu) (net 16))
 (segment (start 88.659999 48.784999) (end 89.555 49.68) (width 0.25) (layer F.Cu) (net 11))
 (segment (start 78.215001 48.784999) (end 88.659999 48.784999) (width 0.25) (layer F.Cu) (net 11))
 (segment (start 76.2 50.8) (end 78.215001 48.784999) (width 0.25) (layer F.Cu) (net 11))
 (segment (start 76.2 48.26) (end 76.2 48.411002) (width 0.25) (layer F.Cu) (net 12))
 (segment (start 76.78 47.68) (end 76.2 48.26) (width 0.25) (layer F.Cu) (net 12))
 (segment (start 89.61 48.26) (end 90.19 47.68) (width 0.25) (layer F.Cu) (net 12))
 (segment (start 76.2 48.26) (end 89.61 48.26) (width 0.25) (layer F.Cu) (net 12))
 (segment (start 86.654999 47.715001) (end 88.69 45.68) (width 0.25) (layer F.Cu) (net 13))
 (segment (start 88.69 45.68) (end 90.19 45.68) (width 0.25) (layer F.Cu) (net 13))
 (segment (start 78.195001 47.715001) (end 86.654999 47.715001) (width 0.25) (layer F.Cu) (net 13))
 (segment (start 76.2 45.72) (end 78.195001 47.715001) (width 0.25) (layer F.Cu) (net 13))
 (segment (start 107.64069 49.68) (end 104.755 49.68) (width 0.25) (layer F.Cu) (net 6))
 (segment (start 108.76069 50.8) (end 107.64069 49.68) (width 0.25) (layer F.Cu) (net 6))
 (segment (start 118.11 50.8) (end 108.76069 50.8) (width 0.25) (layer F.Cu) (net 6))
 (segment (start 108.835 48.26) (end 118.11 48.26) (width 0.25) (layer F.Cu) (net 4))
 (segment (start 106.255 45.68) (end 108.835 48.26) (width 0.25) (layer F.Cu) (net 4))
 (segment (start 104.755 45.68) (end 106.255 45.68) (width 0.25) (layer F.Cu) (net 4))
 (segment (start 105.090002 43.68) (end 104.755 43.68) (width 0.25) (layer F.Cu) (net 3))
 (segment (start 117.82749 45.43749) (end 118.11 45.72) (width 0.25) (layer F.Cu) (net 3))
 (segment (start 116.07 43.68) (end 118.11 45.72) (width 0.25) (layer F.Cu) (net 3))
 (segment (start 105.39 43.68) (end 116.07 43.68) (width 0.25) (layer F.Cu) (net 3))
 (segment (start 79.86 50.11) (end 86.36 50.11) (width 0.25) (layer F.Cu) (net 10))
 (segment (start 87.93 51.68) (end 89.555 51.68) (width 0.25) (layer F.Cu) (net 10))
 (segment (start 86.36 50.11) (end 87.93 51.68) (width 0.25) (layer F.Cu) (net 10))
 (segment (start 79.86 47.475) (end 79.375 46.99) (width 0.25) (layer B.Cu) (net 10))
 (segment (start 79.86 50.11) (end 79.86 47.475) (width 0.25) (layer B.Cu) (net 10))
 (segment (start 79.375 45.8) (end 79.455 45.72) (width 0.25) (layer F.Cu) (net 10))
 (segment (start 79.375 46.99) (end 79.375 45.8) (width 0.25) (layer F.Cu) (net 10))
 (segment (start 100.32 39.8) (end 100.09 40.03) (width 0.25) (layer B.Cu) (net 17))
 (segment (start 102.87 39.8) (end 100.32 39.8) (width 0.25) (layer B.Cu) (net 17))
 (segment (start 111.215 37.7) (end 111.215 36.777002) (width 0.25) (layer F.Cu) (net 17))
 (segment (start 111.215 36.777002) (end 113.067002 34.925) (width 0.25) (layer F.Cu) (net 17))
 (segment (start 116.115 36.939998) (end 116.115 37.7) (width 0.25) (layer F.Cu) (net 17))
 (segment (start 114.100002 34.925) (end 116.115 36.939998) (width 0.25) (layer F.Cu) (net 17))
 (segment (start 113.067002 34.925) (end 114.100002 34.925) (width 0.25) (layer F.Cu) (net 17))
 (segment (start 107.315 37.09826) (end 107.315 38.1) (width 0.25) (layer F.Cu) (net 17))
 (segment (start 109.48826 34.925) (end 107.315 37.09826) (width 0.25) (layer F.Cu) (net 17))
 (segment (start 113.067002 34.925) (end 109.48826 34.925) (width 0.25) (layer F.Cu) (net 17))
 (segment (start 105.615 39.8) (end 102.87 39.8) (width 0.25) (layer B.Cu) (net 17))
 (segment (start 107.315 38.1) (end 105.615 39.8) (width 0.25) (layer B.Cu) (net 17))
 (segment (start 114.415 38.660002) (end 114.415 37.7) (width 0.25) (layer F.Cu) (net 27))
 (segment (start 114.325001 38.750001) (end 114.415 38.660002) (width 0.25) (layer F.Cu) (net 27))
 (segment (start 113.415 38.675) (end 113.490001 38.750001) (width 0.25) (layer F.Cu) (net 27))
 (segment (start 113.490001 38.750001) (end 114.325001 38.750001) (width 0.25) (layer F.Cu) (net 27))
 (segment (start 113.415 37.7) (end 113.415 38.675) (width 0.25) (layer F.Cu) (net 27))
 (segment (start 114.415 38.780685) (end 114.415 37.7) (width 0.25) (layer F.Cu) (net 27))
 (segment (start 115.004315 39.37) (end 114.415 38.780685) (width 0.25) (layer F.Cu) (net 27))
 (segment (start 115.57 39.37) (end 115.004315 39.37) (width 0.25) (layer F.Cu) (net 27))
 (segment (start 114.844999 40.095001) (end 115.57 39.37) (width 0.25) (layer B.Cu) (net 27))
 (segment (start 108.219999 40.095001) (end 114.844999 40.095001) (width 0.25) (layer B.Cu) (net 27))
 (segment (start 99.695 48.62) (end 108.219999 40.095001) (width 0.25) (layer B.Cu) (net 27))
 (segment (start 99.695 49.595) (end 99.695 48.62) (width 0.25) (layer B.Cu) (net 27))
 (segment (start 113.915 36.725) (end 113.915 37.7) (width 0.25) (layer F.Cu) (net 28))
 (segment (start 113.004999 36.649999) (end 113.839999 36.649999) (width 0.25) (layer F.Cu) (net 28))
 (segment (start 113.839999 36.649999) (end 113.915 36.725) (width 0.25) (layer F.Cu) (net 28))
 (segment (start 112.915 36.739998) (end 113.004999 36.649999) (width 0.25) (layer F.Cu) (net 28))
 (segment (start 112.915 37.7) (end 112.915 36.739998) (width 0.25) (layer F.Cu) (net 28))
 (segment (start 112.915 38.675) (end 112.915 37.7) (width 0.25) (layer F.Cu) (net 28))
 (segment (start 112.22 39.37) (end 112.915 38.675) (width 0.25) (layer F.Cu) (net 28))
 (segment (start 110.49 39.37) (end 112.22 39.37) (width 0.25) (layer F.Cu) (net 28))
 (segment (start 108.273232 39.37) (end 98.425 49.218232) (width 0.25) (layer B.Cu) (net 28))
 (segment (start 98.425 49.218232) (end 98.425 49.595) (width 0.25) (layer B.Cu) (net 28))
 (segment (start 110.49 39.37) (end 108.273232 39.37) (width 0.25) (layer B.Cu) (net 28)))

